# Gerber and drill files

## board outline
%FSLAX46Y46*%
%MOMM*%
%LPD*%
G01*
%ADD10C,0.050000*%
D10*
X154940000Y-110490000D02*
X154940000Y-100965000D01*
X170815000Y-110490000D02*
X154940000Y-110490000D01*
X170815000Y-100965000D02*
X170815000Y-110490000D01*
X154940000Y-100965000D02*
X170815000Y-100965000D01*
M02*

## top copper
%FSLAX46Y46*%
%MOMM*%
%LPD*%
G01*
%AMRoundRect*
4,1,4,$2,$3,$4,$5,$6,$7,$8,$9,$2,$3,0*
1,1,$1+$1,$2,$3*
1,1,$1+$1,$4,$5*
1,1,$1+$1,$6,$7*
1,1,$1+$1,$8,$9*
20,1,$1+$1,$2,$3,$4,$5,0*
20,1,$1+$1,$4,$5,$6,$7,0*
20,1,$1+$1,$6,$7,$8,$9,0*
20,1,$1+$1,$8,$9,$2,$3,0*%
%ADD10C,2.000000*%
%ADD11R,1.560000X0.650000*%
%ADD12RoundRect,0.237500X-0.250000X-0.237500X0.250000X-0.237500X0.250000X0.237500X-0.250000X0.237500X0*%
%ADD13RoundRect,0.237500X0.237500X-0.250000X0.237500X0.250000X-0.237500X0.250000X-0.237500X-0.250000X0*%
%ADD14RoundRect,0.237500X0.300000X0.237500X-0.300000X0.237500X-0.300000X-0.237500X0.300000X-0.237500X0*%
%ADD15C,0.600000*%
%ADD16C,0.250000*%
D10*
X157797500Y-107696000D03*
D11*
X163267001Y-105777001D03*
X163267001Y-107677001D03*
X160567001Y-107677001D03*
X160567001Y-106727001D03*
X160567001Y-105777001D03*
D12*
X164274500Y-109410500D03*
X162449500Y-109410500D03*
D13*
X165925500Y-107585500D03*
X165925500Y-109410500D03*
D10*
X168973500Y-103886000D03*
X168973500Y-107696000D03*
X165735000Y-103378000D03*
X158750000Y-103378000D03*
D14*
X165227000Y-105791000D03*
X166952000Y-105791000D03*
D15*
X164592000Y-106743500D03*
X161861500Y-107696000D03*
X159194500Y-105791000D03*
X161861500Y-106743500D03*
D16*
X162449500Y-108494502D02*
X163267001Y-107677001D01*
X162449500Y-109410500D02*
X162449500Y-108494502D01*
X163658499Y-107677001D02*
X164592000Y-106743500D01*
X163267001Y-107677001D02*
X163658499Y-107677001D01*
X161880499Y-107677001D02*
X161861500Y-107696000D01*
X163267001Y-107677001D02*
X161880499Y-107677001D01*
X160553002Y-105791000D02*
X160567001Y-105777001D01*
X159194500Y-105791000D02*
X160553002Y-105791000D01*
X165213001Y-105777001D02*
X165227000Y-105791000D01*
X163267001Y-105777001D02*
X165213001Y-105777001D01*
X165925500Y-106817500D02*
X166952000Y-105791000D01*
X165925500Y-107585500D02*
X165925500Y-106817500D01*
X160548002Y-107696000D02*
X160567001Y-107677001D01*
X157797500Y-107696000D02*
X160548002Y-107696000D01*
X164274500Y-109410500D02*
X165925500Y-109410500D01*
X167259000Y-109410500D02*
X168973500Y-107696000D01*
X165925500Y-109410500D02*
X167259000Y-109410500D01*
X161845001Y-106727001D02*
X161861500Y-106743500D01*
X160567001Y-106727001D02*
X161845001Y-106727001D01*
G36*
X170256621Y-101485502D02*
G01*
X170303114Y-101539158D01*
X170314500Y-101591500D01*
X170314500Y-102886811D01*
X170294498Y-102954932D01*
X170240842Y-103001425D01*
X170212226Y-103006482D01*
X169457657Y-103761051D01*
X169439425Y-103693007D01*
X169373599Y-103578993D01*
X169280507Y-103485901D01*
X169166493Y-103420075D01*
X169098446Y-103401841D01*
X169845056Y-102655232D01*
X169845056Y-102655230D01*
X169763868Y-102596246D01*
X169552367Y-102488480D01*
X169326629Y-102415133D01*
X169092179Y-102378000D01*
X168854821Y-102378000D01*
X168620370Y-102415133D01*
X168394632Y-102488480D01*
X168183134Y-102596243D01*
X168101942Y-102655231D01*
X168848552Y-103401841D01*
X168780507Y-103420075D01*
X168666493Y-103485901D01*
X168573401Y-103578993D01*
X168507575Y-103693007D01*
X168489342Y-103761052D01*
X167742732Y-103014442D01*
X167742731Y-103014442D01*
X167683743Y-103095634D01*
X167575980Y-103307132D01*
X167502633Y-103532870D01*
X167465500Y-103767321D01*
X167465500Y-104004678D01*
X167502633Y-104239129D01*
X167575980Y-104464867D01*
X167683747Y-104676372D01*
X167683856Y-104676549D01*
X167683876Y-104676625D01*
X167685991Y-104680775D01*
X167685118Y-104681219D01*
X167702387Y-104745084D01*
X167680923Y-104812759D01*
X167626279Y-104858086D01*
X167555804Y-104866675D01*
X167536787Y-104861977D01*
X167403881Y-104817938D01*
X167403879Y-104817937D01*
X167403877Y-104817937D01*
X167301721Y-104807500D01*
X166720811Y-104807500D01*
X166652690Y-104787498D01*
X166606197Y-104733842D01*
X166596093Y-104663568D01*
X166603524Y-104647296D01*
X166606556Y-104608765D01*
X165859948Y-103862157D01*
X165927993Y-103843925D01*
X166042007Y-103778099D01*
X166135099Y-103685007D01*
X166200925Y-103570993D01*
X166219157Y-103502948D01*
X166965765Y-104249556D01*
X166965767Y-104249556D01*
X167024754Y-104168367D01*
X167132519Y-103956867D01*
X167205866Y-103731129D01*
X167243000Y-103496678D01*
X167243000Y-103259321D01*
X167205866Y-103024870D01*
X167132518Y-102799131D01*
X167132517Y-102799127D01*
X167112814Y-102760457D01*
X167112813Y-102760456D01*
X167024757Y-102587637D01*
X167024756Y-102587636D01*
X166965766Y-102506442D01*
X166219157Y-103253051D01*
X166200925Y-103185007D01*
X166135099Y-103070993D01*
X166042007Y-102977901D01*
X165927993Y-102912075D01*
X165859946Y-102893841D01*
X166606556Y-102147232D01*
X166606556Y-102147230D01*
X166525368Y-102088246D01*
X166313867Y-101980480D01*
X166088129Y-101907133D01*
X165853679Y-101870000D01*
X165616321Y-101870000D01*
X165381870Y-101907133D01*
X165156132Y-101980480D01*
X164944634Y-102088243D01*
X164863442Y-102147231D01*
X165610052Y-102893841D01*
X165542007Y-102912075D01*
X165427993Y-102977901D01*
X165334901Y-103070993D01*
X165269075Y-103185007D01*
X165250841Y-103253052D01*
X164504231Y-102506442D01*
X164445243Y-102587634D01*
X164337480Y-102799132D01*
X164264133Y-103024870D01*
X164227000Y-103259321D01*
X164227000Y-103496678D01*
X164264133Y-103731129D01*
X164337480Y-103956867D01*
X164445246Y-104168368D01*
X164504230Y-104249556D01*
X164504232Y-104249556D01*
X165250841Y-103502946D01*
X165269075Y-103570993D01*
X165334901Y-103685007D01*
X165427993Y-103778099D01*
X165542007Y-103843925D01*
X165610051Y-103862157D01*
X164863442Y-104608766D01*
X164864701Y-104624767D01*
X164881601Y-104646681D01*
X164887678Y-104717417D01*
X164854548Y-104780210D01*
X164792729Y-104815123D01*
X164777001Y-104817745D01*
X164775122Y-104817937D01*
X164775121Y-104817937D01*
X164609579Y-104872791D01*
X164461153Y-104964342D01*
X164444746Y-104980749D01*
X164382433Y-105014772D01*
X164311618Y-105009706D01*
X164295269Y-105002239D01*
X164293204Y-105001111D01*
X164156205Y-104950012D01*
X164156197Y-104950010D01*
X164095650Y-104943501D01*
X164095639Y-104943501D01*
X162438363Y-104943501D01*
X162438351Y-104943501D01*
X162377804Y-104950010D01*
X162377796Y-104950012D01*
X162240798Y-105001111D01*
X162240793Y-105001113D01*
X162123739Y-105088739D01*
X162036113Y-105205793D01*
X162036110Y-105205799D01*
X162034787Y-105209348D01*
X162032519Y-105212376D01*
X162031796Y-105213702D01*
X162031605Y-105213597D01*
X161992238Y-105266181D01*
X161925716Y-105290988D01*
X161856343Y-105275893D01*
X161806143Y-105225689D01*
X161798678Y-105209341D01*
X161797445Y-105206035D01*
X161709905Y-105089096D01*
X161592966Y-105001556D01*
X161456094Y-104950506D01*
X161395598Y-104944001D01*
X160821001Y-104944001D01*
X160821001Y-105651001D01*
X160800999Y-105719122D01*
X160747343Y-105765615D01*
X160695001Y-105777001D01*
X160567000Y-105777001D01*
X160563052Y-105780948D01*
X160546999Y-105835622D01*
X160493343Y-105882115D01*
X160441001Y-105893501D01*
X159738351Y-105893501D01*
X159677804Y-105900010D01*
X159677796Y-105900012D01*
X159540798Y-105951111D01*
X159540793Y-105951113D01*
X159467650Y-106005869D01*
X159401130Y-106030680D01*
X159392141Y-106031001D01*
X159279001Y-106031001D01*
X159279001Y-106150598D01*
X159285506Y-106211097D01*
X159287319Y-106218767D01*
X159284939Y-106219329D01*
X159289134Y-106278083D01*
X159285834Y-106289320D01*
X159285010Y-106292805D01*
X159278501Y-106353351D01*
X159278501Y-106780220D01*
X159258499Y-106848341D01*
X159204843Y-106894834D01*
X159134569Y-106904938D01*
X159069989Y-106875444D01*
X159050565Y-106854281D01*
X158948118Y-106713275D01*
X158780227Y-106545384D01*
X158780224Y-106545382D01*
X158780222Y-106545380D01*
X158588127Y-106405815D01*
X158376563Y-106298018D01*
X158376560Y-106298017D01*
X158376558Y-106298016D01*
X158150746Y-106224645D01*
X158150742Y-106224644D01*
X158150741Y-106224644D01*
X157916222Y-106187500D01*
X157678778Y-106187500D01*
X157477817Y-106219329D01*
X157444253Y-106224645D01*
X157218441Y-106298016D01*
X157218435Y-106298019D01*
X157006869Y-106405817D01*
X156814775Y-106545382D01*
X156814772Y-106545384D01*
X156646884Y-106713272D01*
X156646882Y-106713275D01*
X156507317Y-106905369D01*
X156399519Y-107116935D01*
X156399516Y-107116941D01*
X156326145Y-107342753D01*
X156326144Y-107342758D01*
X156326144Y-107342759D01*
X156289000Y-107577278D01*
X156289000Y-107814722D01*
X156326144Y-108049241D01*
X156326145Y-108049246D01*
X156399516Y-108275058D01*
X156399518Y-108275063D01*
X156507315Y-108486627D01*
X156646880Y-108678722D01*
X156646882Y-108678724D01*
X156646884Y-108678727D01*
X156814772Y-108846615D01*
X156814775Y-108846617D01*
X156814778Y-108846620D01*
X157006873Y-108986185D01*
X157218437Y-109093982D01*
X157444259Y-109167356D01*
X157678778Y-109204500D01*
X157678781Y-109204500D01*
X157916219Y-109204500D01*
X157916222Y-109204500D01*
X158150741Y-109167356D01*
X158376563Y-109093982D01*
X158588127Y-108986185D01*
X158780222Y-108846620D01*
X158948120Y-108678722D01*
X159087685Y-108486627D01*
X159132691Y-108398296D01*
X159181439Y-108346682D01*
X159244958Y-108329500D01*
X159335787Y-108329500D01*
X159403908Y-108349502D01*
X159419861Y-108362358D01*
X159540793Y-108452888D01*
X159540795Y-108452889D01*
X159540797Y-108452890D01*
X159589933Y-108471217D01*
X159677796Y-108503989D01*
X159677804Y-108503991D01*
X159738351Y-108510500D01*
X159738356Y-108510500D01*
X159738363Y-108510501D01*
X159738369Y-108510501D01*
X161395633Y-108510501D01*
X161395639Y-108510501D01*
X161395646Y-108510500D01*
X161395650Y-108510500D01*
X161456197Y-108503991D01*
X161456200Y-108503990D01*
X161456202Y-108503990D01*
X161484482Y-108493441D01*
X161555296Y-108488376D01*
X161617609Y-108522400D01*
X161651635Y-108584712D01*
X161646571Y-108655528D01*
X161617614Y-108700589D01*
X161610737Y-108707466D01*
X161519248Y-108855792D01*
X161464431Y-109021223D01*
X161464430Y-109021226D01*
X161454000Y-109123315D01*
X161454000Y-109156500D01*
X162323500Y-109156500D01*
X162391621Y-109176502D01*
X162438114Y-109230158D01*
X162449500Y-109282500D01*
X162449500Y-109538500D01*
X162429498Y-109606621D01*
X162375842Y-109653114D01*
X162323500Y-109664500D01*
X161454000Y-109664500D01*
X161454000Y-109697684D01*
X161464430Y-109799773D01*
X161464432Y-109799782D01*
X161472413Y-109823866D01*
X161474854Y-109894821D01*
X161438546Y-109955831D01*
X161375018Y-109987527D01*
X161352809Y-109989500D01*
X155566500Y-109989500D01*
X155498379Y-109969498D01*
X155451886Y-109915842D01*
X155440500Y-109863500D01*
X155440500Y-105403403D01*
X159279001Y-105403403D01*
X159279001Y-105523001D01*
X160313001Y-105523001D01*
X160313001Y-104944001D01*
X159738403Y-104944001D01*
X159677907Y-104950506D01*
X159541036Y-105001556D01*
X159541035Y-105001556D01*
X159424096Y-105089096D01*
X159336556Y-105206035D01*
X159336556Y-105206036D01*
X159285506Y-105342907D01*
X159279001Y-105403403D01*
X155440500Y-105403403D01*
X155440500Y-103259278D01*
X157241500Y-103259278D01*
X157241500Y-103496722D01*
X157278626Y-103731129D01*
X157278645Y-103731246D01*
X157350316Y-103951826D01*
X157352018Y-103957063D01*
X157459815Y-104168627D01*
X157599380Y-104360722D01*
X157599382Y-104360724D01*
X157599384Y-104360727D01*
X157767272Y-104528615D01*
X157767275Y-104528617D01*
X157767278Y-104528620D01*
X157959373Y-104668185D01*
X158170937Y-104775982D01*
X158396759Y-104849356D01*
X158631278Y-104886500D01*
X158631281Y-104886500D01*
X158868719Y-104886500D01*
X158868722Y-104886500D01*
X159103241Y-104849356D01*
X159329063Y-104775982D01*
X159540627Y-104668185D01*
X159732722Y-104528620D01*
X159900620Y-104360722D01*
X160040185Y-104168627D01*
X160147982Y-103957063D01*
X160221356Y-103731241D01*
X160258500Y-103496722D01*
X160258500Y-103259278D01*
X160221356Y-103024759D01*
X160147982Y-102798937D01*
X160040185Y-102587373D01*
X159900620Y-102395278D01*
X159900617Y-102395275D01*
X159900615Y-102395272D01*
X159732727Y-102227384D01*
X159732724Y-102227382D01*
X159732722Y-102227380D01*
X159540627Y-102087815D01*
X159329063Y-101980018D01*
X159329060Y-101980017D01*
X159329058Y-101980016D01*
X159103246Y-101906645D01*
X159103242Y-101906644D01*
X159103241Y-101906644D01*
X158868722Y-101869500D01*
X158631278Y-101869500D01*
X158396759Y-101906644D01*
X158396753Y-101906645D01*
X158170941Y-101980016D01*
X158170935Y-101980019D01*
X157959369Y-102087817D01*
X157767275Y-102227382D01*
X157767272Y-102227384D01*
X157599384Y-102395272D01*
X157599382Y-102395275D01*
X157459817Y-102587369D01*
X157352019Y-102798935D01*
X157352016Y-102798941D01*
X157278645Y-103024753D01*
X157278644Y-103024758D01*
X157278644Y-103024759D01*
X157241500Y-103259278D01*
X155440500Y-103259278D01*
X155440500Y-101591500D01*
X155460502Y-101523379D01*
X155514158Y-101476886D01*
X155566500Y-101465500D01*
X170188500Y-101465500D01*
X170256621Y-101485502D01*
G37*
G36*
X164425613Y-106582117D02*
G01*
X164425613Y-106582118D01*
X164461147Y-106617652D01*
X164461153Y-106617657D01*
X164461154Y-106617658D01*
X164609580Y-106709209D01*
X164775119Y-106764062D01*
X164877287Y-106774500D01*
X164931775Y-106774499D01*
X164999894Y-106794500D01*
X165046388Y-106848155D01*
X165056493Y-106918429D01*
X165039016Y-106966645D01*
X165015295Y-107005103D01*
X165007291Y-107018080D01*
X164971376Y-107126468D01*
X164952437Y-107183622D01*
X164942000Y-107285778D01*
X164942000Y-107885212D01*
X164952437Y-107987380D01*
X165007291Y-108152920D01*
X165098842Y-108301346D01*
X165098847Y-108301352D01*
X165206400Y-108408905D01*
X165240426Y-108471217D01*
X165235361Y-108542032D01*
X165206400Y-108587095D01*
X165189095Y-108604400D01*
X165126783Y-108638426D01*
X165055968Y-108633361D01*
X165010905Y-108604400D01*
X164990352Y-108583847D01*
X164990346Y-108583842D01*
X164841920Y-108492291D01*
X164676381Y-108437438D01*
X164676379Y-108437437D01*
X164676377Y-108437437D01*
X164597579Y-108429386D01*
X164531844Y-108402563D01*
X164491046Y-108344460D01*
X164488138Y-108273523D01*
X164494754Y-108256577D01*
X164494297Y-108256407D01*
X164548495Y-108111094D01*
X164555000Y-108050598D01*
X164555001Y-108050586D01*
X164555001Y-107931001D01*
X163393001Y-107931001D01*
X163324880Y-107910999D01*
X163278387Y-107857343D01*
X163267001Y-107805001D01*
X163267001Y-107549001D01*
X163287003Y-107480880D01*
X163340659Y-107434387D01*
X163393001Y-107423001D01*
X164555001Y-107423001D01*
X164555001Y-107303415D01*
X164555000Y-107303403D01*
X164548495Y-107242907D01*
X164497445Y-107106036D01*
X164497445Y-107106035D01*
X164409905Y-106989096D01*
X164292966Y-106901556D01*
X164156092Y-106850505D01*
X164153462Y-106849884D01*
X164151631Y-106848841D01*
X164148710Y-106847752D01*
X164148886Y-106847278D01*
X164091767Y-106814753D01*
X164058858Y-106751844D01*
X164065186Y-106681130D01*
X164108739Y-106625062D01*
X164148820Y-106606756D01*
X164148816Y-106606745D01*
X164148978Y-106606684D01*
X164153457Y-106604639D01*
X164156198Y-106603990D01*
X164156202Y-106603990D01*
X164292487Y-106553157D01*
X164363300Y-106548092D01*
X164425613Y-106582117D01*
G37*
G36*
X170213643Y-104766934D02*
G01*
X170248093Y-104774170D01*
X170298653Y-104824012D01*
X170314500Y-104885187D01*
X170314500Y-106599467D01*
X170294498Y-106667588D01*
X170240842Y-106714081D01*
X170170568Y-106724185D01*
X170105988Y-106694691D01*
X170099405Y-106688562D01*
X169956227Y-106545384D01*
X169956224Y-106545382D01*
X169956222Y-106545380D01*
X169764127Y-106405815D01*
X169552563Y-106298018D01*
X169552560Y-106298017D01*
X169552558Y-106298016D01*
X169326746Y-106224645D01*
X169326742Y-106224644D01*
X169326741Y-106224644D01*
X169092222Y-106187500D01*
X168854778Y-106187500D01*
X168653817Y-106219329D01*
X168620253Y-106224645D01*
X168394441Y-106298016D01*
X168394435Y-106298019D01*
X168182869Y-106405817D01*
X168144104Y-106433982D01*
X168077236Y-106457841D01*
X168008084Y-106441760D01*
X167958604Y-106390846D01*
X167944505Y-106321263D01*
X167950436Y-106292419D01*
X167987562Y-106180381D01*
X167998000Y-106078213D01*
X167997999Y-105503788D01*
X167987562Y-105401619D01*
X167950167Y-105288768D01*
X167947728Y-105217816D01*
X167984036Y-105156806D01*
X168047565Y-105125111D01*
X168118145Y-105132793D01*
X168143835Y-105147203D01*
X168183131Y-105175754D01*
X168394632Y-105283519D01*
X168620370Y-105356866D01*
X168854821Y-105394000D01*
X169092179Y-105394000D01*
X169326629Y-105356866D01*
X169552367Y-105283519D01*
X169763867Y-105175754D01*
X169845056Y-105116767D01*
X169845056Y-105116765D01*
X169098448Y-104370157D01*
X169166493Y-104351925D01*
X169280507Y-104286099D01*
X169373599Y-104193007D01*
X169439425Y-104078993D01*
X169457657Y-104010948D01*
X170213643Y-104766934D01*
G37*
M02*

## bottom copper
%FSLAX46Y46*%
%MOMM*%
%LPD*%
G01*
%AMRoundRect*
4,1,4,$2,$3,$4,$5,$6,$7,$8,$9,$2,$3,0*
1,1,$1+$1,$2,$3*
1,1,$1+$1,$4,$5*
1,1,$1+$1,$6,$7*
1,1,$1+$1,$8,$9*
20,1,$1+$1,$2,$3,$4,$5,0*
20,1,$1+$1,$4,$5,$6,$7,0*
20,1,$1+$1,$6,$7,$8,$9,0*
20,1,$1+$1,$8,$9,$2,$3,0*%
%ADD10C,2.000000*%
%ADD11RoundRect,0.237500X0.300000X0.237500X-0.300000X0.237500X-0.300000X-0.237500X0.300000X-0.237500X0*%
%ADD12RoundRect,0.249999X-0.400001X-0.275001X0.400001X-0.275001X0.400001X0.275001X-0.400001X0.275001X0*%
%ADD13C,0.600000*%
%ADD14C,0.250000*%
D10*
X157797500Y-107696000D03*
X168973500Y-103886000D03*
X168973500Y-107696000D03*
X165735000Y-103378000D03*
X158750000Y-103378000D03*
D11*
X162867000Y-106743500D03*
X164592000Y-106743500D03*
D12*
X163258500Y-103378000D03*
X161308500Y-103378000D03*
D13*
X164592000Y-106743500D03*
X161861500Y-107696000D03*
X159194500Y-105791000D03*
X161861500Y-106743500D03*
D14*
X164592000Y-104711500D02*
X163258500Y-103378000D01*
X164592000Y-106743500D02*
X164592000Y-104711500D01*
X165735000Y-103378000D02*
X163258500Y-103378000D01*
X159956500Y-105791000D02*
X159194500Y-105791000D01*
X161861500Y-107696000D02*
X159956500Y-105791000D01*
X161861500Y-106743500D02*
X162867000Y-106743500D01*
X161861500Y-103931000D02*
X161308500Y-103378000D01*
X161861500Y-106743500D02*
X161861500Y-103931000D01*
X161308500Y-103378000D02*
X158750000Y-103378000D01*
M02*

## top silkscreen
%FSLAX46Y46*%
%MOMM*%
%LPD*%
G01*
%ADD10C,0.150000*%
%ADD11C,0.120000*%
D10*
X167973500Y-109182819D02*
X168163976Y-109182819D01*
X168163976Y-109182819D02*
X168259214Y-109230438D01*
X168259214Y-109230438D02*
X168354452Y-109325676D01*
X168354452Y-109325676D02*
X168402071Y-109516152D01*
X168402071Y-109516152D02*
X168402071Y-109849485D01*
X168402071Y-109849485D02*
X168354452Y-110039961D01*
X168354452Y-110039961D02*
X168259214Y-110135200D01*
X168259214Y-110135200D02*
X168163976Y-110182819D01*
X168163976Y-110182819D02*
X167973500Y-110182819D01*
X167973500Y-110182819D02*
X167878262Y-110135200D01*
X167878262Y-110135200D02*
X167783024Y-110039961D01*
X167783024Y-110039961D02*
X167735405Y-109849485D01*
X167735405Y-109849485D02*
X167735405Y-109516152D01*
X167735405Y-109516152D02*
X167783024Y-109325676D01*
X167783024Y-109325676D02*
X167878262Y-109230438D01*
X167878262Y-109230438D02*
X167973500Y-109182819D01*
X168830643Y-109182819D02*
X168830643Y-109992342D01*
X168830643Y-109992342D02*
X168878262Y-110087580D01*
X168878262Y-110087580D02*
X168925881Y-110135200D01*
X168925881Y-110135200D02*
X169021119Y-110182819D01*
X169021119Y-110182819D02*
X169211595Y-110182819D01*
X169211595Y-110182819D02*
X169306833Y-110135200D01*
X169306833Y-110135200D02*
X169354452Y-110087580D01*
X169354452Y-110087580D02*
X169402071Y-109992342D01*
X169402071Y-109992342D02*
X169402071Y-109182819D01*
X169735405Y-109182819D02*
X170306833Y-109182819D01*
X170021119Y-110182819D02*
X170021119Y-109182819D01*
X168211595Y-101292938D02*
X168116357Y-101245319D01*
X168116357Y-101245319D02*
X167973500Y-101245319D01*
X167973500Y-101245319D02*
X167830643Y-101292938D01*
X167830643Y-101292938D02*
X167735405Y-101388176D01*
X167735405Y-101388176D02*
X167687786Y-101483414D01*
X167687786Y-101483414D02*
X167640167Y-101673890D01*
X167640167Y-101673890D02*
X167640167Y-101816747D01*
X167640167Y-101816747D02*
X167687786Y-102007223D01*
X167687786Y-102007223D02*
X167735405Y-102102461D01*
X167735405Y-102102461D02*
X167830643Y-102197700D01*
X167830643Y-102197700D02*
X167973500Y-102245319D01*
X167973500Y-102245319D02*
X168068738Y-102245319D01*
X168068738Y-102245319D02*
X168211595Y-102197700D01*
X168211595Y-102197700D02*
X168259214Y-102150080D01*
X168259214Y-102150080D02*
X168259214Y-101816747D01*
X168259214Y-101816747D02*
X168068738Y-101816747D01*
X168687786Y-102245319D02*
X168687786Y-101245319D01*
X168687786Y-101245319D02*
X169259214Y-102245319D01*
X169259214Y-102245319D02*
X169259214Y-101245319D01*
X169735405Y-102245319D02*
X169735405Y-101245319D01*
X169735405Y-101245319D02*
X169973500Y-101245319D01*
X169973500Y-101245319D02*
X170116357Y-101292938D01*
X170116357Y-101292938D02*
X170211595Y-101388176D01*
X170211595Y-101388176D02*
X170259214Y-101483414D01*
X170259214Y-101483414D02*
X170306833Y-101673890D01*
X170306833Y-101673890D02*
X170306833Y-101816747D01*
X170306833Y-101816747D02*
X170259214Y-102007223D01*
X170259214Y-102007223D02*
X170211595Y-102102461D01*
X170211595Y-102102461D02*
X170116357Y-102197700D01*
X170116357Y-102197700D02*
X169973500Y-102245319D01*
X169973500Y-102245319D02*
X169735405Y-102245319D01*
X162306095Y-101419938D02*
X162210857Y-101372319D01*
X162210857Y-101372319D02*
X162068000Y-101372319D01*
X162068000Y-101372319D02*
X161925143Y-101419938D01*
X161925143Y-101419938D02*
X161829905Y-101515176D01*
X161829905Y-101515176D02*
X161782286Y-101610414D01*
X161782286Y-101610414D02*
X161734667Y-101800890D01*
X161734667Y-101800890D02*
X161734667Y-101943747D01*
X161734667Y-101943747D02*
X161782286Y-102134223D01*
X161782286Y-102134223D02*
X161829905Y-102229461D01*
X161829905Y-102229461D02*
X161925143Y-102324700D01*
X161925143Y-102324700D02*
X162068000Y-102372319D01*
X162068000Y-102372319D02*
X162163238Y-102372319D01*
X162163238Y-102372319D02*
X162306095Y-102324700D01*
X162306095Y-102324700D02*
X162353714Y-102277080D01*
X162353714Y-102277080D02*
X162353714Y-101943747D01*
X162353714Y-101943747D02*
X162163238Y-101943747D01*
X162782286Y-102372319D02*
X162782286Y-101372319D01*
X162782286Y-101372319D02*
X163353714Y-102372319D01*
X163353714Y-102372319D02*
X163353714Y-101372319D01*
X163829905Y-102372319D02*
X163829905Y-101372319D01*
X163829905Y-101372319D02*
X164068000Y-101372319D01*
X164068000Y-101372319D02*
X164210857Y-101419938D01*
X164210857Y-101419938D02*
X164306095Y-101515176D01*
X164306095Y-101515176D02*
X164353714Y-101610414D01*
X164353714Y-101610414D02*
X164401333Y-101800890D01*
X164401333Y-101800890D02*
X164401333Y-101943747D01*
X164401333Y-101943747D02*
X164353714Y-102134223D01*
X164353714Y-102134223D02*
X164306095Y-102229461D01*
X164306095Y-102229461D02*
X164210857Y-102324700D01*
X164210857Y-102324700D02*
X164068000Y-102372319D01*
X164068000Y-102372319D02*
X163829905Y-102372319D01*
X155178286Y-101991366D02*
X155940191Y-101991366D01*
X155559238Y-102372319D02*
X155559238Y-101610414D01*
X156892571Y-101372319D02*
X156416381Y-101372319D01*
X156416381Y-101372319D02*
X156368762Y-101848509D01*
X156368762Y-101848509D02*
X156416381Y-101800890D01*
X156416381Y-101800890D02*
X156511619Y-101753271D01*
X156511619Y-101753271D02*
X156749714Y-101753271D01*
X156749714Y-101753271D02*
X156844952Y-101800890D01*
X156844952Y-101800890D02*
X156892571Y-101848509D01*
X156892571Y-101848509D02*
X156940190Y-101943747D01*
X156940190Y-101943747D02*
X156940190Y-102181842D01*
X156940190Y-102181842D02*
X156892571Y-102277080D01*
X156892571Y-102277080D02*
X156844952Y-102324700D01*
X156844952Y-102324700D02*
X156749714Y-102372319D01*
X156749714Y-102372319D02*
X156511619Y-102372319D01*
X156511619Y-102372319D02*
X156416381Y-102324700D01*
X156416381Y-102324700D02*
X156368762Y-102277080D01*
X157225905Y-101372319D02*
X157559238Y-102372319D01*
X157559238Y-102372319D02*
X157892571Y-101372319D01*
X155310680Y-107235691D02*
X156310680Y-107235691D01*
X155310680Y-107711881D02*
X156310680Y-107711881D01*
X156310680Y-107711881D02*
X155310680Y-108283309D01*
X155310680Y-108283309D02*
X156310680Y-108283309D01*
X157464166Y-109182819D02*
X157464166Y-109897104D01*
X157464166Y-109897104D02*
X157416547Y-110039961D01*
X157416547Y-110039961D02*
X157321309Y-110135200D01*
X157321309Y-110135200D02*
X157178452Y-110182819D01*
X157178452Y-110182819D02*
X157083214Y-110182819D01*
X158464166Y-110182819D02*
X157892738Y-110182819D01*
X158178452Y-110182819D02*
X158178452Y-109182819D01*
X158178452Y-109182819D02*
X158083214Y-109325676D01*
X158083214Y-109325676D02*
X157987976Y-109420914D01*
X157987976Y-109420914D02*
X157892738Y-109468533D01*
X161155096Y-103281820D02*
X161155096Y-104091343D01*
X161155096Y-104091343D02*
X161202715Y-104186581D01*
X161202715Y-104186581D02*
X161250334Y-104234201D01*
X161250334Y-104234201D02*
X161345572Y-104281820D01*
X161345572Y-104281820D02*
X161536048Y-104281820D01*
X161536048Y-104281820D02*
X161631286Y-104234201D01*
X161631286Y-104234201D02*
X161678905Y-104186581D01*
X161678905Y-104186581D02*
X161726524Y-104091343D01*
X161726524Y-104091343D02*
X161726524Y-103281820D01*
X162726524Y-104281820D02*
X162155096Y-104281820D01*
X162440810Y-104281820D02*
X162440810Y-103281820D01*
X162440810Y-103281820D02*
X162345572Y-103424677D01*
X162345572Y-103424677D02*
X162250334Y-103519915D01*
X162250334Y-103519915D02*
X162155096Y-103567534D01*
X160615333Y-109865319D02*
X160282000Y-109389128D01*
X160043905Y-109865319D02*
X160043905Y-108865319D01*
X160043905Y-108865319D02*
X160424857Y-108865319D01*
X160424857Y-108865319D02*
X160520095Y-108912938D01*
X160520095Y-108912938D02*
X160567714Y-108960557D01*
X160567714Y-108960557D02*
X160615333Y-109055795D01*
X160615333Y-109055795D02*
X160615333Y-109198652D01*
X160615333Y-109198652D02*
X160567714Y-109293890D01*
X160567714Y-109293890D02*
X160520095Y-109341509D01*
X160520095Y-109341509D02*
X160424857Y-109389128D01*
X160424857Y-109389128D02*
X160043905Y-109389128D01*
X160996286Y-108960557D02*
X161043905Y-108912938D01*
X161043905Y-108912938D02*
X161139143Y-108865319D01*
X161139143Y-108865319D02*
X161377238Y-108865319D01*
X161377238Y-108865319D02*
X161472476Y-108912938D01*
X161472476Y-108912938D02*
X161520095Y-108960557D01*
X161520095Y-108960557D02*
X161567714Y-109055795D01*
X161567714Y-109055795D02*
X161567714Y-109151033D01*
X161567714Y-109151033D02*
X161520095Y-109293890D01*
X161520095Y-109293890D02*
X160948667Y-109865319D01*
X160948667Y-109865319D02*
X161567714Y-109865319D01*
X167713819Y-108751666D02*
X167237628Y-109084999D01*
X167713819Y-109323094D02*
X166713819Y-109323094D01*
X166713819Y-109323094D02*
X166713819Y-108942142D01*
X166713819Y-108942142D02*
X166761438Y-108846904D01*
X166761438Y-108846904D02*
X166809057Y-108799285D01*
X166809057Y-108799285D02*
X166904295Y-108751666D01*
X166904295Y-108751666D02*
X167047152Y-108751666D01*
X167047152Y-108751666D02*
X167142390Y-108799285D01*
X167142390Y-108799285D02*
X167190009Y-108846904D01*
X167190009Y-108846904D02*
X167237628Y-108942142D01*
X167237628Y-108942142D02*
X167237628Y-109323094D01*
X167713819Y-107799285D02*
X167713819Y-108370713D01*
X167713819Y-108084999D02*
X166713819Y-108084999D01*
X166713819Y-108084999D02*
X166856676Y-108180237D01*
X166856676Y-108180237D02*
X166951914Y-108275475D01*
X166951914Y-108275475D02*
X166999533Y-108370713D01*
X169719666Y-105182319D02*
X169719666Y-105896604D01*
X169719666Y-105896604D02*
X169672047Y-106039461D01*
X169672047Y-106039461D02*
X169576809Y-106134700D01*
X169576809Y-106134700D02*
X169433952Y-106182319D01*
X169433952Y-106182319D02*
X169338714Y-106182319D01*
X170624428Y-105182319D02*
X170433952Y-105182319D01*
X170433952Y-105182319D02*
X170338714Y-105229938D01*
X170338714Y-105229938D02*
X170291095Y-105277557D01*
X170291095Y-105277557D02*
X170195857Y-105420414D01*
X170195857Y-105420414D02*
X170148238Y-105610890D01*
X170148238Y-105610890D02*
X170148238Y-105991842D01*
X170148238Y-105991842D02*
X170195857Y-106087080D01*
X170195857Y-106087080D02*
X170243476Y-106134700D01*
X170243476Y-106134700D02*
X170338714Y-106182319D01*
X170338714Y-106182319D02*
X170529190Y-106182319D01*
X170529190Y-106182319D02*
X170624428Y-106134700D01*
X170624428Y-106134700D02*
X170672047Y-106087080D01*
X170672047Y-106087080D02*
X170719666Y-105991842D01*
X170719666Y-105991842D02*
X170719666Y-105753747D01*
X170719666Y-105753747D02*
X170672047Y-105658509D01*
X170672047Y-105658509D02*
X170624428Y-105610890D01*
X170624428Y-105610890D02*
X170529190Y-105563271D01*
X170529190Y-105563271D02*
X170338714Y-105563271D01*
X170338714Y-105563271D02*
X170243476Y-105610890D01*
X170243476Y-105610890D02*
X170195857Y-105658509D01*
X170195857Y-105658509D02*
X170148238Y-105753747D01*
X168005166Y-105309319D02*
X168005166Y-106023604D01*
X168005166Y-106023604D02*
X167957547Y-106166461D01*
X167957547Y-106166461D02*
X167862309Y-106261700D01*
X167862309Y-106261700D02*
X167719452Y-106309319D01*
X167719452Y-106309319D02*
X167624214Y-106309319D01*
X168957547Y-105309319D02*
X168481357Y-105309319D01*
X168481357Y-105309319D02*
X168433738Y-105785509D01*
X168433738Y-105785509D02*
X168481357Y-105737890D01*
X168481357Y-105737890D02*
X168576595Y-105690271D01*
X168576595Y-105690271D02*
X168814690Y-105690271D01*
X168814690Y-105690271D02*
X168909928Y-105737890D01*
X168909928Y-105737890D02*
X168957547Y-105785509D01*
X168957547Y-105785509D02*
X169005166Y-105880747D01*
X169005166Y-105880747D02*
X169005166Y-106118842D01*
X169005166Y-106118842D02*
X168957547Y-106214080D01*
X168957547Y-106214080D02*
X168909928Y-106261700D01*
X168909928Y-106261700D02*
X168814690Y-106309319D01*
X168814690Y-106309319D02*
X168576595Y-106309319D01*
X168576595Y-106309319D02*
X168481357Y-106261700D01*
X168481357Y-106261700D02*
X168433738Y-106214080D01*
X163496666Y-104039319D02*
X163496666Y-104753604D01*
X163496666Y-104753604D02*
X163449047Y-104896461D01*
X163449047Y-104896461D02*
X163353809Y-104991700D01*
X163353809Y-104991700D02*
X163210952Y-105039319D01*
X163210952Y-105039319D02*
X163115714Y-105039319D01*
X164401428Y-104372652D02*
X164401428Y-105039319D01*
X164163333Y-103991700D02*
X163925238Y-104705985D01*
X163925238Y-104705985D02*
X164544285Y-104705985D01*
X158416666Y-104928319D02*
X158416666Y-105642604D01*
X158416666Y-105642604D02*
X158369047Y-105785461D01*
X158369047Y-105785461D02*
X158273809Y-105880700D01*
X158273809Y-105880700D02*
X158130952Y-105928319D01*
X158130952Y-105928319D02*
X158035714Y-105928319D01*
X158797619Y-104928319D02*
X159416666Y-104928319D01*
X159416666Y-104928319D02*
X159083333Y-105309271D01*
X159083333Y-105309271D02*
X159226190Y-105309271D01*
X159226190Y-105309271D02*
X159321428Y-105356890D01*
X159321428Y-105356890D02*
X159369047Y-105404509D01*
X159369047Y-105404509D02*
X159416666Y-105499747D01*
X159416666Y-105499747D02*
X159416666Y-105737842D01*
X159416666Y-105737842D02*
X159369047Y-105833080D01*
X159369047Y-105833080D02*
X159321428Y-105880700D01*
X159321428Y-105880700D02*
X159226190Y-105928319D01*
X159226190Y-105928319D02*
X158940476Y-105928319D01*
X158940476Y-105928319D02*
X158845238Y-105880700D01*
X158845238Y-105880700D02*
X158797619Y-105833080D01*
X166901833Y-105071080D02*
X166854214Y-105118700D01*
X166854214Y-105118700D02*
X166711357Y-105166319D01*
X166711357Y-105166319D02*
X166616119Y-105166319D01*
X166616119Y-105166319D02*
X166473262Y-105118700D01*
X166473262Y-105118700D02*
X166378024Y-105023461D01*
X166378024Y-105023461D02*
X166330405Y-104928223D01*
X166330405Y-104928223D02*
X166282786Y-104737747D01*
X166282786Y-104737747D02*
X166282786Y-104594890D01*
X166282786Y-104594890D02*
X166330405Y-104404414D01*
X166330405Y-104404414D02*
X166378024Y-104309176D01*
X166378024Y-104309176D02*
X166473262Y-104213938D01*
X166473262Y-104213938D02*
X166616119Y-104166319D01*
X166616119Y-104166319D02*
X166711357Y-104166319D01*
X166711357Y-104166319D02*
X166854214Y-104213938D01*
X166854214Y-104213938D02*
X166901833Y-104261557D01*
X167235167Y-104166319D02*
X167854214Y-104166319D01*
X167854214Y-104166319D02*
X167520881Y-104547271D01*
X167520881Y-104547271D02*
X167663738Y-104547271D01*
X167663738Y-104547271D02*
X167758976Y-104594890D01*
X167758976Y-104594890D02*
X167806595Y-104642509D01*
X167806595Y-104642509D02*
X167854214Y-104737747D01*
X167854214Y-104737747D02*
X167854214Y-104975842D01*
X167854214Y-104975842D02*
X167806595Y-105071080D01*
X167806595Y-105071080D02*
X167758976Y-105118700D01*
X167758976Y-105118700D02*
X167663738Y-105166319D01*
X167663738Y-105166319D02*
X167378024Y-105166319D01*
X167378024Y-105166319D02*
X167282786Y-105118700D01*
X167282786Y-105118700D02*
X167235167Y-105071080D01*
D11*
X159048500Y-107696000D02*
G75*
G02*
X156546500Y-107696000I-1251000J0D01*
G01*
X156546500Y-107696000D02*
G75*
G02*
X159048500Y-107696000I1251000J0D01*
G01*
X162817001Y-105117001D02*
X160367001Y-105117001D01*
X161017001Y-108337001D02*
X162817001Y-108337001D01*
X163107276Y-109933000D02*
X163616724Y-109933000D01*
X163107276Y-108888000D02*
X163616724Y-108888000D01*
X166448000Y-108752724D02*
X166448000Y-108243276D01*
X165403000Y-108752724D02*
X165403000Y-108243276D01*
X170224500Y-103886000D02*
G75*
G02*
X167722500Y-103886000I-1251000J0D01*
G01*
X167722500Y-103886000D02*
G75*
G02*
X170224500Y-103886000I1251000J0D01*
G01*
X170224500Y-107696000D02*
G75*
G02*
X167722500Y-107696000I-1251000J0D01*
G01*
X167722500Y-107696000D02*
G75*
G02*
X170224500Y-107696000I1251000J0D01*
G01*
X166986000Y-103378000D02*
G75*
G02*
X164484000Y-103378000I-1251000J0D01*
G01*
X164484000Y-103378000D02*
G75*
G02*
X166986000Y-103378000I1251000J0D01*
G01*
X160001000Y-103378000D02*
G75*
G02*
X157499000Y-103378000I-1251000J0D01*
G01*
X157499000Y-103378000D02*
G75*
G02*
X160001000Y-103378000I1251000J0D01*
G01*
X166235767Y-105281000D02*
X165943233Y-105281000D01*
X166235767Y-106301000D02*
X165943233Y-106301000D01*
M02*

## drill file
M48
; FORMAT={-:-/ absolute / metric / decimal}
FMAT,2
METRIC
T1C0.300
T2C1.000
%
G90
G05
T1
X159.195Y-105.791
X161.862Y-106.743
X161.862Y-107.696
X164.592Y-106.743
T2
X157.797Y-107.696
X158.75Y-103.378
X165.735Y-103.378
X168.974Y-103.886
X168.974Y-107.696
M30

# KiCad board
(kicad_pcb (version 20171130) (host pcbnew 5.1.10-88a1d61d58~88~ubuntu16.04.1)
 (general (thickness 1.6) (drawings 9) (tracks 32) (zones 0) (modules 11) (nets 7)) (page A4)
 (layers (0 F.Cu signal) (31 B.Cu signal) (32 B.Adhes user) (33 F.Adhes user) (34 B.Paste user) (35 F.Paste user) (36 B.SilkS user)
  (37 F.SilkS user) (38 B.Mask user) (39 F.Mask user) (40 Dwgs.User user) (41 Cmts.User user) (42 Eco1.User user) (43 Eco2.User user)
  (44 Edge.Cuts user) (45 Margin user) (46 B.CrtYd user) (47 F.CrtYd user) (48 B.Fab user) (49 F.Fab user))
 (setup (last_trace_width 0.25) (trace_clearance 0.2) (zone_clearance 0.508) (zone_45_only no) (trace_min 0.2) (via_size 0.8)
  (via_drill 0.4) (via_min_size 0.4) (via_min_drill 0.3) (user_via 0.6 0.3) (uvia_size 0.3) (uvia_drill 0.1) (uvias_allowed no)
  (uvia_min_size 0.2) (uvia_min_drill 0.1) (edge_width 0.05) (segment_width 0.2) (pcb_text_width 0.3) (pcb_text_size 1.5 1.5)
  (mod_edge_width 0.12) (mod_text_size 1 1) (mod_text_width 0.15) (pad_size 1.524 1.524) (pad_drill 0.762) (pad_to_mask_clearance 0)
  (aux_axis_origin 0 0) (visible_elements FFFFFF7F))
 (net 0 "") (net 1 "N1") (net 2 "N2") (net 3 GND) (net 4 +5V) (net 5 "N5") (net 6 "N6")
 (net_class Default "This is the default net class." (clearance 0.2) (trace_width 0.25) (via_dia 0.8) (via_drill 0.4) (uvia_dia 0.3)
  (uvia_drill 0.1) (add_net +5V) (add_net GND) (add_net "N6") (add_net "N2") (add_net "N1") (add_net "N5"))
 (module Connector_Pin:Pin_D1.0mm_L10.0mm (layer F.Cu) (at 157.7975 107.696)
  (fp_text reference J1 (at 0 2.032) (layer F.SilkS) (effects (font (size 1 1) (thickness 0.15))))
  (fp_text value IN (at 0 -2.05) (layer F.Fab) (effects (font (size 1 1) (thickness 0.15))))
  (fp_circle (center 0 0) (end 1.25 0.05) (layer F.SilkS) (width 0.12))
  (pad 1 thru_hole circle (at 0 0) (size 2 2) (drill 1) (layers *.Cu *.Mask) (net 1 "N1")))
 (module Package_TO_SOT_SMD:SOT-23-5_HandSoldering (layer F.Cu) (at 161.917001 106.727001)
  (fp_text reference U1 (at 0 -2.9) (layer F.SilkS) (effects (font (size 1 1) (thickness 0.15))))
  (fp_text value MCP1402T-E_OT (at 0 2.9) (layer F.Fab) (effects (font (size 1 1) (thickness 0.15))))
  (fp_line (start 0.9 -1.61) (end -1.55 -1.61) (layer F.SilkS) (width 0.12))
  (fp_line (start -0.9 1.61) (end 0.9 1.61) (layer F.SilkS) (width 0.12))
  (pad 5 smd rect (at 1.35 -0.95) (size 1.56 0.65) (layers F.Cu F.Paste F.Mask) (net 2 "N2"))
  (pad 4 smd rect (at 1.35 0.95) (size 1.56 0.65) (layers F.Cu F.Paste F.Mask) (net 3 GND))
  (pad 3 smd rect (at -1.35 0.95) (size 1.56 0.65) (layers F.Cu F.Paste F.Mask) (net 1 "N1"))
  (pad 2 smd rect (at -1.35 0) (size 1.56 0.65) (layers F.Cu F.Paste F.Mask) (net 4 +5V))
  (pad 1 smd rect (at -1.35 -0.95) (size 1.56 0.65) (layers F.Cu F.Paste F.Mask) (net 3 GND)))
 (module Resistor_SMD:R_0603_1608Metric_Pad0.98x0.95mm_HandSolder (layer F.Cu) (at 163.362 109.4105)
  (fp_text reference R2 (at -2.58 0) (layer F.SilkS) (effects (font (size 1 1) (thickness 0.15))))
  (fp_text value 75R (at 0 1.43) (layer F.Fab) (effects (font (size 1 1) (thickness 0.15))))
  (fp_line (start -0.254724 0.5225) (end 0.254724 0.5225) (layer F.SilkS) (width 0.12))
  (fp_line (start -0.254724 -0.5225) (end 0.254724 -0.5225) (layer F.SilkS) (width 0.12))
  (pad 2 smd roundrect (at 0.9125 0) (size 0.975 0.95) (layers F.Cu F.Paste F.Mask) (roundrect_rratio 0.25) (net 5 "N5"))
  (pad 1 smd roundrect (at -0.9125 0) (size 0.975 0.95) (layers F.Cu F.Paste F.Mask) (roundrect_rratio 0.25) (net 3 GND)))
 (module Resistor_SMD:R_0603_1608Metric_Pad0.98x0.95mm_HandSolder (layer F.Cu) (at 165.9255 108.498 90)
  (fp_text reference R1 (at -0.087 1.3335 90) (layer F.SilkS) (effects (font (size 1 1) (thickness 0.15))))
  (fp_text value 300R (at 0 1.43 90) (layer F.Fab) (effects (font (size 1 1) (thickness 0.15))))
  (fp_line (start -0.254724 0.5225) (end 0.254724 0.5225) (layer F.SilkS) (width 0.12))
  (fp_line (start -0.254724 -0.5225) (end 0.254724 -0.5225) (layer F.SilkS) (width 0.12))
  (pad 2 smd roundrect (at 0.9125 0 90) (size 0.975 0.95) (layers F.Cu F.Paste F.Mask) (roundrect_rratio 0.25) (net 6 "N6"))
  (pad 1 smd roundrect (at -0.9125 0 90) (size 0.975 0.95) (layers F.Cu F.Paste F.Mask) (roundrect_rratio 0.25) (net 5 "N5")))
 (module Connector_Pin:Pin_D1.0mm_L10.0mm (layer F.Cu) (at 168.9735 103.886)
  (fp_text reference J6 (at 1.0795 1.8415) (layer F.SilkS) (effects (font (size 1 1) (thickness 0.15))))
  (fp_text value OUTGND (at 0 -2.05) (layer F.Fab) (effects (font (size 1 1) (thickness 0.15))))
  (fp_circle (center 0 0) (end 1.25 0.05) (layer F.SilkS) (width 0.12))
  (pad 1 thru_hole circle (at 0 0) (size 2 2) (drill 1) (layers *.Cu *.Mask) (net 3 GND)))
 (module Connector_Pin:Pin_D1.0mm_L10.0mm (layer F.Cu) (at 168.9735 107.696)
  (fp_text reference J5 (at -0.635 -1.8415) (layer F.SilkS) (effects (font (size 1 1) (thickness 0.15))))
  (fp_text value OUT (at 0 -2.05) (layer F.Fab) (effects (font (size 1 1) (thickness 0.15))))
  (fp_circle (center 0 0) (end 1.25 0.05) (layer F.SilkS) (width 0.12))
  (pad 1 thru_hole circle (at 0 0) (size 2 2) (drill 1) (layers *.Cu *.Mask) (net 5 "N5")))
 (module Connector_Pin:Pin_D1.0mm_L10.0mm (layer F.Cu) (at 165.735 103.378)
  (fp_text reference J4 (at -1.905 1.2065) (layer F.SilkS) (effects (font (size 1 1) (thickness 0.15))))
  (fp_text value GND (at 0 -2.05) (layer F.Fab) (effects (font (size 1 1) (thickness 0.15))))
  (fp_circle (center 0 0) (end 1.25 0.05) (layer F.SilkS) (width 0.12))
  (pad 1 thru_hole circle (at 0 0) (size 2 2) (drill 1) (layers *.Cu *.Mask) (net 3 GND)))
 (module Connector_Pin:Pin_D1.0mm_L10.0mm (layer F.Cu) (at 158.75 103.378)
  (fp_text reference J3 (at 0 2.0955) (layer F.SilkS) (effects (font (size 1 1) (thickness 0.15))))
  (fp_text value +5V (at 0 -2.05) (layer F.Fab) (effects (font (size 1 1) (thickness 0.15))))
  (fp_circle (center 0 0) (end 1.25 0.05) (layer F.SilkS) (width 0.12))
  (pad 1 thru_hole circle (at 0 0) (size 2 2) (drill 1) (layers *.Cu *.Mask) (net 4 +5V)))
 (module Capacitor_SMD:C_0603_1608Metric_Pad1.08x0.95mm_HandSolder (layer F.Cu) (at 166.0895 105.791 180)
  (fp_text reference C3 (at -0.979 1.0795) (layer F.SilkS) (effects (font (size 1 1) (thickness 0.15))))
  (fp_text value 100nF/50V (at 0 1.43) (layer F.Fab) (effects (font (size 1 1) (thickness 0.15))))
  (fp_line (start -0.146267 0.51) (end 0.146267 0.51) (layer F.SilkS) (width 0.12))
  (fp_line (start -0.146267 -0.51) (end 0.146267 -0.51) (layer F.SilkS) (width 0.12))
  (pad 2 smd roundrect (at 0.8625 0 180) (size 1.075 0.95) (layers F.Cu F.Paste F.Mask) (roundrect_rratio 0.25) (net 2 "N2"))
  (pad 1 smd roundrect (at -0.8625 0 180) (size 1.075 0.95) (layers F.Cu F.Paste F.Mask) (roundrect_rratio 0.25) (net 6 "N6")))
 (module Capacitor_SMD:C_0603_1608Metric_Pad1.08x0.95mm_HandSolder (layer B.Cu) (at 163.7295 106.7435 180)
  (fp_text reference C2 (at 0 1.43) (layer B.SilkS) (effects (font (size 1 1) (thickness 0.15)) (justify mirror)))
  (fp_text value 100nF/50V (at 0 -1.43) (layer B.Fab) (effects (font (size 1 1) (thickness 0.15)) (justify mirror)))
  (pad 2 smd roundrect (at 0.8625 0 180) (size 1.075 0.95) (layers B.Cu B.Paste B.Mask) (roundrect_rratio 0.25) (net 4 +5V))
  (pad 1 smd roundrect (at -0.8625 0 180) (size 1.075 0.95) (layers B.Cu B.Paste B.Mask) (roundrect_rratio 0.25) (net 3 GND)))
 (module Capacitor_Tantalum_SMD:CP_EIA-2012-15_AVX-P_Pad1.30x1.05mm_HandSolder (layer B.Cu) (at 162.2835 103.378)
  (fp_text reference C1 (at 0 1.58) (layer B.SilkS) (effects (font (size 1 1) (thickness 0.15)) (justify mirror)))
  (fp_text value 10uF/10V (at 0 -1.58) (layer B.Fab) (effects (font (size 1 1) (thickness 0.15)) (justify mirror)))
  (pad 2 smd roundrect (at 0.975 0) (size 1.3 1.05) (layers B.Cu B.Paste B.Mask) (roundrect_rratio 0.2380942857142857) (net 3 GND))
  (pad 1 smd roundrect (at -0.975 0) (size 1.3 1.05) (layers B.Cu B.Paste B.Mask) (roundrect_rratio 0.2380942857142857) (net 4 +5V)))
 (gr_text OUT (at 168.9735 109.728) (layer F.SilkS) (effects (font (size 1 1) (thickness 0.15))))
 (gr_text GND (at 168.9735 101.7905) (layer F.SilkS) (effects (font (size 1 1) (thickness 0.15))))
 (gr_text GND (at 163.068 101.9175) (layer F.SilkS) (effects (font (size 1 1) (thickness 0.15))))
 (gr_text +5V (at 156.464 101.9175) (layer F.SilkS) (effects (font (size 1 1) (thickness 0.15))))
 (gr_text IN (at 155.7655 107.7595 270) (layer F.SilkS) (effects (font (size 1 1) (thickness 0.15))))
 (gr_line (start 154.94 110.49) (end 154.94 100.965) (layer Edge.Cuts) (width 0.05))
 (gr_line (start 170.815 110.49) (end 154.94 110.49) (layer Edge.Cuts) (width 0.05))
 (gr_line (start 170.815 100.965) (end 170.815 110.49) (layer Edge.Cuts) (width 0.05))
 (gr_line (start 154.94 100.965) (end 170.815 100.965) (layer Edge.Cuts) (width 0.05))
 (segment (start 162.4495 108.494502) (end 163.267001 107.677001) (width 0.25) (layer F.Cu) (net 3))
 (segment (start 162.4495 109.4105) (end 162.4495 108.494502) (width 0.25) (layer F.Cu) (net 3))
 (segment (start 164.592 104.7115) (end 163.2585 103.378) (width 0.25) (layer B.Cu) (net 3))
 (segment (start 164.592 106.7435) (end 164.592 104.7115) (width 0.25) (layer B.Cu) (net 3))
 (segment (start 165.735 103.378) (end 163.2585 103.378) (width 0.25) (layer B.Cu) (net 3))
 (via (at 164.592 106.7435) (size 0.6) (drill 0.3) (layers F.Cu B.Cu) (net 3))
 (segment (start 163.658499 107.677001) (end 164.592 106.7435) (width 0.25) (layer F.Cu) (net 3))
 (segment (start 163.267001 107.677001) (end 163.658499 107.677001) (width 0.25) (layer F.Cu) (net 3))
 (via (at 161.8615 107.696) (size 0.6) (drill 0.3) (layers F.Cu B.Cu) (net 3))
 (segment (start 161.880499 107.677001) (end 161.8615 107.696) (width 0.25) (layer F.Cu) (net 3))
 (segment (start 163.267001 107.677001) (end 161.880499 107.677001) (width 0.25) (layer F.Cu) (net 3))
 (via (at 159.1945 105.791) (size 0.6) (drill 0.3) (layers F.Cu B.Cu) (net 3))
 (segment (start 159.9565 105.791) (end 159.1945 105.791) (width 0.25) (layer B.Cu) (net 3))
 (segment (start 161.8615 107.696) (end 159.9565 105.791) (width 0.25) (layer B.Cu) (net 3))
 (segment (start 160.553002 105.791) (end 160.567001 105.777001) (width 0.25) (layer F.Cu) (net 3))
 (segment (start 159.1945 105.791) (end 160.553002 105.791) (width 0.25) (layer F.Cu) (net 3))
 (segment (start 165.213001 105.777001) (end 165.227 105.791) (width 0.25) (layer F.Cu) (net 2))
 (segment (start 163.267001 105.777001) (end 165.213001 105.777001) (width 0.25) (layer F.Cu) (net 2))
 (segment (start 165.9255 106.8175) (end 166.952 105.791) (width 0.25) (layer F.Cu) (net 6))
 (segment (start 165.9255 107.5855) (end 165.9255 106.8175) (width 0.25) (layer F.Cu) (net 6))
 (segment (start 160.548002 107.696) (end 160.567001 107.677001) (width 0.25) (layer F.Cu) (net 1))
 (segment (start 157.7975 107.696) (end 160.548002 107.696) (width 0.25) (layer F.Cu) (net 1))
 (segment (start 164.2745 109.4105) (end 165.9255 109.4105) (width 0.25) (layer F.Cu) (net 5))
 (segment (start 167.259 109.4105) (end 168.9735 107.696) (width 0.25) (layer F.Cu) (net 5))
 (segment (start 165.9255 109.4105) (end 167.259 109.4105) (width 0.25) (layer F.Cu) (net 5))
 (via (at 161.8615 106.7435) (size 0.6) (drill 0.3) (layers F.Cu B.Cu) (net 4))
 (segment (start 161.845001 106.727001) (end 161.8615 106.7435) (width 0.25) (layer F.Cu) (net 4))
 (segment (start 160.567001 106.727001) (end 161.845001 106.727001) (width 0.25) (layer F.Cu) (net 4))
 (segment (start 161.8615 106.7435) (end 162.867 106.7435) (width 0.25) (layer B.Cu) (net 4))
 (segment (start 161.8615 103.931) (end 161.3085 103.378) (width 0.25) (layer B.Cu) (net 4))
 (segment (start 161.8615 106.7435) (end 161.8615 103.931) (width 0.25) (layer B.Cu) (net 4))
 (segment (start 161.3085 103.378) (end 158.75 103.378) (width 0.25) (layer B.Cu) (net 4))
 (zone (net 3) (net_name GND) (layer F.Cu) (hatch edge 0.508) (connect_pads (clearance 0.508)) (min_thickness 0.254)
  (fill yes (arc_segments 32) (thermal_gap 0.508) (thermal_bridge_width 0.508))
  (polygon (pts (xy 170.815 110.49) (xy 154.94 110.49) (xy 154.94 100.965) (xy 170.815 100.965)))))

